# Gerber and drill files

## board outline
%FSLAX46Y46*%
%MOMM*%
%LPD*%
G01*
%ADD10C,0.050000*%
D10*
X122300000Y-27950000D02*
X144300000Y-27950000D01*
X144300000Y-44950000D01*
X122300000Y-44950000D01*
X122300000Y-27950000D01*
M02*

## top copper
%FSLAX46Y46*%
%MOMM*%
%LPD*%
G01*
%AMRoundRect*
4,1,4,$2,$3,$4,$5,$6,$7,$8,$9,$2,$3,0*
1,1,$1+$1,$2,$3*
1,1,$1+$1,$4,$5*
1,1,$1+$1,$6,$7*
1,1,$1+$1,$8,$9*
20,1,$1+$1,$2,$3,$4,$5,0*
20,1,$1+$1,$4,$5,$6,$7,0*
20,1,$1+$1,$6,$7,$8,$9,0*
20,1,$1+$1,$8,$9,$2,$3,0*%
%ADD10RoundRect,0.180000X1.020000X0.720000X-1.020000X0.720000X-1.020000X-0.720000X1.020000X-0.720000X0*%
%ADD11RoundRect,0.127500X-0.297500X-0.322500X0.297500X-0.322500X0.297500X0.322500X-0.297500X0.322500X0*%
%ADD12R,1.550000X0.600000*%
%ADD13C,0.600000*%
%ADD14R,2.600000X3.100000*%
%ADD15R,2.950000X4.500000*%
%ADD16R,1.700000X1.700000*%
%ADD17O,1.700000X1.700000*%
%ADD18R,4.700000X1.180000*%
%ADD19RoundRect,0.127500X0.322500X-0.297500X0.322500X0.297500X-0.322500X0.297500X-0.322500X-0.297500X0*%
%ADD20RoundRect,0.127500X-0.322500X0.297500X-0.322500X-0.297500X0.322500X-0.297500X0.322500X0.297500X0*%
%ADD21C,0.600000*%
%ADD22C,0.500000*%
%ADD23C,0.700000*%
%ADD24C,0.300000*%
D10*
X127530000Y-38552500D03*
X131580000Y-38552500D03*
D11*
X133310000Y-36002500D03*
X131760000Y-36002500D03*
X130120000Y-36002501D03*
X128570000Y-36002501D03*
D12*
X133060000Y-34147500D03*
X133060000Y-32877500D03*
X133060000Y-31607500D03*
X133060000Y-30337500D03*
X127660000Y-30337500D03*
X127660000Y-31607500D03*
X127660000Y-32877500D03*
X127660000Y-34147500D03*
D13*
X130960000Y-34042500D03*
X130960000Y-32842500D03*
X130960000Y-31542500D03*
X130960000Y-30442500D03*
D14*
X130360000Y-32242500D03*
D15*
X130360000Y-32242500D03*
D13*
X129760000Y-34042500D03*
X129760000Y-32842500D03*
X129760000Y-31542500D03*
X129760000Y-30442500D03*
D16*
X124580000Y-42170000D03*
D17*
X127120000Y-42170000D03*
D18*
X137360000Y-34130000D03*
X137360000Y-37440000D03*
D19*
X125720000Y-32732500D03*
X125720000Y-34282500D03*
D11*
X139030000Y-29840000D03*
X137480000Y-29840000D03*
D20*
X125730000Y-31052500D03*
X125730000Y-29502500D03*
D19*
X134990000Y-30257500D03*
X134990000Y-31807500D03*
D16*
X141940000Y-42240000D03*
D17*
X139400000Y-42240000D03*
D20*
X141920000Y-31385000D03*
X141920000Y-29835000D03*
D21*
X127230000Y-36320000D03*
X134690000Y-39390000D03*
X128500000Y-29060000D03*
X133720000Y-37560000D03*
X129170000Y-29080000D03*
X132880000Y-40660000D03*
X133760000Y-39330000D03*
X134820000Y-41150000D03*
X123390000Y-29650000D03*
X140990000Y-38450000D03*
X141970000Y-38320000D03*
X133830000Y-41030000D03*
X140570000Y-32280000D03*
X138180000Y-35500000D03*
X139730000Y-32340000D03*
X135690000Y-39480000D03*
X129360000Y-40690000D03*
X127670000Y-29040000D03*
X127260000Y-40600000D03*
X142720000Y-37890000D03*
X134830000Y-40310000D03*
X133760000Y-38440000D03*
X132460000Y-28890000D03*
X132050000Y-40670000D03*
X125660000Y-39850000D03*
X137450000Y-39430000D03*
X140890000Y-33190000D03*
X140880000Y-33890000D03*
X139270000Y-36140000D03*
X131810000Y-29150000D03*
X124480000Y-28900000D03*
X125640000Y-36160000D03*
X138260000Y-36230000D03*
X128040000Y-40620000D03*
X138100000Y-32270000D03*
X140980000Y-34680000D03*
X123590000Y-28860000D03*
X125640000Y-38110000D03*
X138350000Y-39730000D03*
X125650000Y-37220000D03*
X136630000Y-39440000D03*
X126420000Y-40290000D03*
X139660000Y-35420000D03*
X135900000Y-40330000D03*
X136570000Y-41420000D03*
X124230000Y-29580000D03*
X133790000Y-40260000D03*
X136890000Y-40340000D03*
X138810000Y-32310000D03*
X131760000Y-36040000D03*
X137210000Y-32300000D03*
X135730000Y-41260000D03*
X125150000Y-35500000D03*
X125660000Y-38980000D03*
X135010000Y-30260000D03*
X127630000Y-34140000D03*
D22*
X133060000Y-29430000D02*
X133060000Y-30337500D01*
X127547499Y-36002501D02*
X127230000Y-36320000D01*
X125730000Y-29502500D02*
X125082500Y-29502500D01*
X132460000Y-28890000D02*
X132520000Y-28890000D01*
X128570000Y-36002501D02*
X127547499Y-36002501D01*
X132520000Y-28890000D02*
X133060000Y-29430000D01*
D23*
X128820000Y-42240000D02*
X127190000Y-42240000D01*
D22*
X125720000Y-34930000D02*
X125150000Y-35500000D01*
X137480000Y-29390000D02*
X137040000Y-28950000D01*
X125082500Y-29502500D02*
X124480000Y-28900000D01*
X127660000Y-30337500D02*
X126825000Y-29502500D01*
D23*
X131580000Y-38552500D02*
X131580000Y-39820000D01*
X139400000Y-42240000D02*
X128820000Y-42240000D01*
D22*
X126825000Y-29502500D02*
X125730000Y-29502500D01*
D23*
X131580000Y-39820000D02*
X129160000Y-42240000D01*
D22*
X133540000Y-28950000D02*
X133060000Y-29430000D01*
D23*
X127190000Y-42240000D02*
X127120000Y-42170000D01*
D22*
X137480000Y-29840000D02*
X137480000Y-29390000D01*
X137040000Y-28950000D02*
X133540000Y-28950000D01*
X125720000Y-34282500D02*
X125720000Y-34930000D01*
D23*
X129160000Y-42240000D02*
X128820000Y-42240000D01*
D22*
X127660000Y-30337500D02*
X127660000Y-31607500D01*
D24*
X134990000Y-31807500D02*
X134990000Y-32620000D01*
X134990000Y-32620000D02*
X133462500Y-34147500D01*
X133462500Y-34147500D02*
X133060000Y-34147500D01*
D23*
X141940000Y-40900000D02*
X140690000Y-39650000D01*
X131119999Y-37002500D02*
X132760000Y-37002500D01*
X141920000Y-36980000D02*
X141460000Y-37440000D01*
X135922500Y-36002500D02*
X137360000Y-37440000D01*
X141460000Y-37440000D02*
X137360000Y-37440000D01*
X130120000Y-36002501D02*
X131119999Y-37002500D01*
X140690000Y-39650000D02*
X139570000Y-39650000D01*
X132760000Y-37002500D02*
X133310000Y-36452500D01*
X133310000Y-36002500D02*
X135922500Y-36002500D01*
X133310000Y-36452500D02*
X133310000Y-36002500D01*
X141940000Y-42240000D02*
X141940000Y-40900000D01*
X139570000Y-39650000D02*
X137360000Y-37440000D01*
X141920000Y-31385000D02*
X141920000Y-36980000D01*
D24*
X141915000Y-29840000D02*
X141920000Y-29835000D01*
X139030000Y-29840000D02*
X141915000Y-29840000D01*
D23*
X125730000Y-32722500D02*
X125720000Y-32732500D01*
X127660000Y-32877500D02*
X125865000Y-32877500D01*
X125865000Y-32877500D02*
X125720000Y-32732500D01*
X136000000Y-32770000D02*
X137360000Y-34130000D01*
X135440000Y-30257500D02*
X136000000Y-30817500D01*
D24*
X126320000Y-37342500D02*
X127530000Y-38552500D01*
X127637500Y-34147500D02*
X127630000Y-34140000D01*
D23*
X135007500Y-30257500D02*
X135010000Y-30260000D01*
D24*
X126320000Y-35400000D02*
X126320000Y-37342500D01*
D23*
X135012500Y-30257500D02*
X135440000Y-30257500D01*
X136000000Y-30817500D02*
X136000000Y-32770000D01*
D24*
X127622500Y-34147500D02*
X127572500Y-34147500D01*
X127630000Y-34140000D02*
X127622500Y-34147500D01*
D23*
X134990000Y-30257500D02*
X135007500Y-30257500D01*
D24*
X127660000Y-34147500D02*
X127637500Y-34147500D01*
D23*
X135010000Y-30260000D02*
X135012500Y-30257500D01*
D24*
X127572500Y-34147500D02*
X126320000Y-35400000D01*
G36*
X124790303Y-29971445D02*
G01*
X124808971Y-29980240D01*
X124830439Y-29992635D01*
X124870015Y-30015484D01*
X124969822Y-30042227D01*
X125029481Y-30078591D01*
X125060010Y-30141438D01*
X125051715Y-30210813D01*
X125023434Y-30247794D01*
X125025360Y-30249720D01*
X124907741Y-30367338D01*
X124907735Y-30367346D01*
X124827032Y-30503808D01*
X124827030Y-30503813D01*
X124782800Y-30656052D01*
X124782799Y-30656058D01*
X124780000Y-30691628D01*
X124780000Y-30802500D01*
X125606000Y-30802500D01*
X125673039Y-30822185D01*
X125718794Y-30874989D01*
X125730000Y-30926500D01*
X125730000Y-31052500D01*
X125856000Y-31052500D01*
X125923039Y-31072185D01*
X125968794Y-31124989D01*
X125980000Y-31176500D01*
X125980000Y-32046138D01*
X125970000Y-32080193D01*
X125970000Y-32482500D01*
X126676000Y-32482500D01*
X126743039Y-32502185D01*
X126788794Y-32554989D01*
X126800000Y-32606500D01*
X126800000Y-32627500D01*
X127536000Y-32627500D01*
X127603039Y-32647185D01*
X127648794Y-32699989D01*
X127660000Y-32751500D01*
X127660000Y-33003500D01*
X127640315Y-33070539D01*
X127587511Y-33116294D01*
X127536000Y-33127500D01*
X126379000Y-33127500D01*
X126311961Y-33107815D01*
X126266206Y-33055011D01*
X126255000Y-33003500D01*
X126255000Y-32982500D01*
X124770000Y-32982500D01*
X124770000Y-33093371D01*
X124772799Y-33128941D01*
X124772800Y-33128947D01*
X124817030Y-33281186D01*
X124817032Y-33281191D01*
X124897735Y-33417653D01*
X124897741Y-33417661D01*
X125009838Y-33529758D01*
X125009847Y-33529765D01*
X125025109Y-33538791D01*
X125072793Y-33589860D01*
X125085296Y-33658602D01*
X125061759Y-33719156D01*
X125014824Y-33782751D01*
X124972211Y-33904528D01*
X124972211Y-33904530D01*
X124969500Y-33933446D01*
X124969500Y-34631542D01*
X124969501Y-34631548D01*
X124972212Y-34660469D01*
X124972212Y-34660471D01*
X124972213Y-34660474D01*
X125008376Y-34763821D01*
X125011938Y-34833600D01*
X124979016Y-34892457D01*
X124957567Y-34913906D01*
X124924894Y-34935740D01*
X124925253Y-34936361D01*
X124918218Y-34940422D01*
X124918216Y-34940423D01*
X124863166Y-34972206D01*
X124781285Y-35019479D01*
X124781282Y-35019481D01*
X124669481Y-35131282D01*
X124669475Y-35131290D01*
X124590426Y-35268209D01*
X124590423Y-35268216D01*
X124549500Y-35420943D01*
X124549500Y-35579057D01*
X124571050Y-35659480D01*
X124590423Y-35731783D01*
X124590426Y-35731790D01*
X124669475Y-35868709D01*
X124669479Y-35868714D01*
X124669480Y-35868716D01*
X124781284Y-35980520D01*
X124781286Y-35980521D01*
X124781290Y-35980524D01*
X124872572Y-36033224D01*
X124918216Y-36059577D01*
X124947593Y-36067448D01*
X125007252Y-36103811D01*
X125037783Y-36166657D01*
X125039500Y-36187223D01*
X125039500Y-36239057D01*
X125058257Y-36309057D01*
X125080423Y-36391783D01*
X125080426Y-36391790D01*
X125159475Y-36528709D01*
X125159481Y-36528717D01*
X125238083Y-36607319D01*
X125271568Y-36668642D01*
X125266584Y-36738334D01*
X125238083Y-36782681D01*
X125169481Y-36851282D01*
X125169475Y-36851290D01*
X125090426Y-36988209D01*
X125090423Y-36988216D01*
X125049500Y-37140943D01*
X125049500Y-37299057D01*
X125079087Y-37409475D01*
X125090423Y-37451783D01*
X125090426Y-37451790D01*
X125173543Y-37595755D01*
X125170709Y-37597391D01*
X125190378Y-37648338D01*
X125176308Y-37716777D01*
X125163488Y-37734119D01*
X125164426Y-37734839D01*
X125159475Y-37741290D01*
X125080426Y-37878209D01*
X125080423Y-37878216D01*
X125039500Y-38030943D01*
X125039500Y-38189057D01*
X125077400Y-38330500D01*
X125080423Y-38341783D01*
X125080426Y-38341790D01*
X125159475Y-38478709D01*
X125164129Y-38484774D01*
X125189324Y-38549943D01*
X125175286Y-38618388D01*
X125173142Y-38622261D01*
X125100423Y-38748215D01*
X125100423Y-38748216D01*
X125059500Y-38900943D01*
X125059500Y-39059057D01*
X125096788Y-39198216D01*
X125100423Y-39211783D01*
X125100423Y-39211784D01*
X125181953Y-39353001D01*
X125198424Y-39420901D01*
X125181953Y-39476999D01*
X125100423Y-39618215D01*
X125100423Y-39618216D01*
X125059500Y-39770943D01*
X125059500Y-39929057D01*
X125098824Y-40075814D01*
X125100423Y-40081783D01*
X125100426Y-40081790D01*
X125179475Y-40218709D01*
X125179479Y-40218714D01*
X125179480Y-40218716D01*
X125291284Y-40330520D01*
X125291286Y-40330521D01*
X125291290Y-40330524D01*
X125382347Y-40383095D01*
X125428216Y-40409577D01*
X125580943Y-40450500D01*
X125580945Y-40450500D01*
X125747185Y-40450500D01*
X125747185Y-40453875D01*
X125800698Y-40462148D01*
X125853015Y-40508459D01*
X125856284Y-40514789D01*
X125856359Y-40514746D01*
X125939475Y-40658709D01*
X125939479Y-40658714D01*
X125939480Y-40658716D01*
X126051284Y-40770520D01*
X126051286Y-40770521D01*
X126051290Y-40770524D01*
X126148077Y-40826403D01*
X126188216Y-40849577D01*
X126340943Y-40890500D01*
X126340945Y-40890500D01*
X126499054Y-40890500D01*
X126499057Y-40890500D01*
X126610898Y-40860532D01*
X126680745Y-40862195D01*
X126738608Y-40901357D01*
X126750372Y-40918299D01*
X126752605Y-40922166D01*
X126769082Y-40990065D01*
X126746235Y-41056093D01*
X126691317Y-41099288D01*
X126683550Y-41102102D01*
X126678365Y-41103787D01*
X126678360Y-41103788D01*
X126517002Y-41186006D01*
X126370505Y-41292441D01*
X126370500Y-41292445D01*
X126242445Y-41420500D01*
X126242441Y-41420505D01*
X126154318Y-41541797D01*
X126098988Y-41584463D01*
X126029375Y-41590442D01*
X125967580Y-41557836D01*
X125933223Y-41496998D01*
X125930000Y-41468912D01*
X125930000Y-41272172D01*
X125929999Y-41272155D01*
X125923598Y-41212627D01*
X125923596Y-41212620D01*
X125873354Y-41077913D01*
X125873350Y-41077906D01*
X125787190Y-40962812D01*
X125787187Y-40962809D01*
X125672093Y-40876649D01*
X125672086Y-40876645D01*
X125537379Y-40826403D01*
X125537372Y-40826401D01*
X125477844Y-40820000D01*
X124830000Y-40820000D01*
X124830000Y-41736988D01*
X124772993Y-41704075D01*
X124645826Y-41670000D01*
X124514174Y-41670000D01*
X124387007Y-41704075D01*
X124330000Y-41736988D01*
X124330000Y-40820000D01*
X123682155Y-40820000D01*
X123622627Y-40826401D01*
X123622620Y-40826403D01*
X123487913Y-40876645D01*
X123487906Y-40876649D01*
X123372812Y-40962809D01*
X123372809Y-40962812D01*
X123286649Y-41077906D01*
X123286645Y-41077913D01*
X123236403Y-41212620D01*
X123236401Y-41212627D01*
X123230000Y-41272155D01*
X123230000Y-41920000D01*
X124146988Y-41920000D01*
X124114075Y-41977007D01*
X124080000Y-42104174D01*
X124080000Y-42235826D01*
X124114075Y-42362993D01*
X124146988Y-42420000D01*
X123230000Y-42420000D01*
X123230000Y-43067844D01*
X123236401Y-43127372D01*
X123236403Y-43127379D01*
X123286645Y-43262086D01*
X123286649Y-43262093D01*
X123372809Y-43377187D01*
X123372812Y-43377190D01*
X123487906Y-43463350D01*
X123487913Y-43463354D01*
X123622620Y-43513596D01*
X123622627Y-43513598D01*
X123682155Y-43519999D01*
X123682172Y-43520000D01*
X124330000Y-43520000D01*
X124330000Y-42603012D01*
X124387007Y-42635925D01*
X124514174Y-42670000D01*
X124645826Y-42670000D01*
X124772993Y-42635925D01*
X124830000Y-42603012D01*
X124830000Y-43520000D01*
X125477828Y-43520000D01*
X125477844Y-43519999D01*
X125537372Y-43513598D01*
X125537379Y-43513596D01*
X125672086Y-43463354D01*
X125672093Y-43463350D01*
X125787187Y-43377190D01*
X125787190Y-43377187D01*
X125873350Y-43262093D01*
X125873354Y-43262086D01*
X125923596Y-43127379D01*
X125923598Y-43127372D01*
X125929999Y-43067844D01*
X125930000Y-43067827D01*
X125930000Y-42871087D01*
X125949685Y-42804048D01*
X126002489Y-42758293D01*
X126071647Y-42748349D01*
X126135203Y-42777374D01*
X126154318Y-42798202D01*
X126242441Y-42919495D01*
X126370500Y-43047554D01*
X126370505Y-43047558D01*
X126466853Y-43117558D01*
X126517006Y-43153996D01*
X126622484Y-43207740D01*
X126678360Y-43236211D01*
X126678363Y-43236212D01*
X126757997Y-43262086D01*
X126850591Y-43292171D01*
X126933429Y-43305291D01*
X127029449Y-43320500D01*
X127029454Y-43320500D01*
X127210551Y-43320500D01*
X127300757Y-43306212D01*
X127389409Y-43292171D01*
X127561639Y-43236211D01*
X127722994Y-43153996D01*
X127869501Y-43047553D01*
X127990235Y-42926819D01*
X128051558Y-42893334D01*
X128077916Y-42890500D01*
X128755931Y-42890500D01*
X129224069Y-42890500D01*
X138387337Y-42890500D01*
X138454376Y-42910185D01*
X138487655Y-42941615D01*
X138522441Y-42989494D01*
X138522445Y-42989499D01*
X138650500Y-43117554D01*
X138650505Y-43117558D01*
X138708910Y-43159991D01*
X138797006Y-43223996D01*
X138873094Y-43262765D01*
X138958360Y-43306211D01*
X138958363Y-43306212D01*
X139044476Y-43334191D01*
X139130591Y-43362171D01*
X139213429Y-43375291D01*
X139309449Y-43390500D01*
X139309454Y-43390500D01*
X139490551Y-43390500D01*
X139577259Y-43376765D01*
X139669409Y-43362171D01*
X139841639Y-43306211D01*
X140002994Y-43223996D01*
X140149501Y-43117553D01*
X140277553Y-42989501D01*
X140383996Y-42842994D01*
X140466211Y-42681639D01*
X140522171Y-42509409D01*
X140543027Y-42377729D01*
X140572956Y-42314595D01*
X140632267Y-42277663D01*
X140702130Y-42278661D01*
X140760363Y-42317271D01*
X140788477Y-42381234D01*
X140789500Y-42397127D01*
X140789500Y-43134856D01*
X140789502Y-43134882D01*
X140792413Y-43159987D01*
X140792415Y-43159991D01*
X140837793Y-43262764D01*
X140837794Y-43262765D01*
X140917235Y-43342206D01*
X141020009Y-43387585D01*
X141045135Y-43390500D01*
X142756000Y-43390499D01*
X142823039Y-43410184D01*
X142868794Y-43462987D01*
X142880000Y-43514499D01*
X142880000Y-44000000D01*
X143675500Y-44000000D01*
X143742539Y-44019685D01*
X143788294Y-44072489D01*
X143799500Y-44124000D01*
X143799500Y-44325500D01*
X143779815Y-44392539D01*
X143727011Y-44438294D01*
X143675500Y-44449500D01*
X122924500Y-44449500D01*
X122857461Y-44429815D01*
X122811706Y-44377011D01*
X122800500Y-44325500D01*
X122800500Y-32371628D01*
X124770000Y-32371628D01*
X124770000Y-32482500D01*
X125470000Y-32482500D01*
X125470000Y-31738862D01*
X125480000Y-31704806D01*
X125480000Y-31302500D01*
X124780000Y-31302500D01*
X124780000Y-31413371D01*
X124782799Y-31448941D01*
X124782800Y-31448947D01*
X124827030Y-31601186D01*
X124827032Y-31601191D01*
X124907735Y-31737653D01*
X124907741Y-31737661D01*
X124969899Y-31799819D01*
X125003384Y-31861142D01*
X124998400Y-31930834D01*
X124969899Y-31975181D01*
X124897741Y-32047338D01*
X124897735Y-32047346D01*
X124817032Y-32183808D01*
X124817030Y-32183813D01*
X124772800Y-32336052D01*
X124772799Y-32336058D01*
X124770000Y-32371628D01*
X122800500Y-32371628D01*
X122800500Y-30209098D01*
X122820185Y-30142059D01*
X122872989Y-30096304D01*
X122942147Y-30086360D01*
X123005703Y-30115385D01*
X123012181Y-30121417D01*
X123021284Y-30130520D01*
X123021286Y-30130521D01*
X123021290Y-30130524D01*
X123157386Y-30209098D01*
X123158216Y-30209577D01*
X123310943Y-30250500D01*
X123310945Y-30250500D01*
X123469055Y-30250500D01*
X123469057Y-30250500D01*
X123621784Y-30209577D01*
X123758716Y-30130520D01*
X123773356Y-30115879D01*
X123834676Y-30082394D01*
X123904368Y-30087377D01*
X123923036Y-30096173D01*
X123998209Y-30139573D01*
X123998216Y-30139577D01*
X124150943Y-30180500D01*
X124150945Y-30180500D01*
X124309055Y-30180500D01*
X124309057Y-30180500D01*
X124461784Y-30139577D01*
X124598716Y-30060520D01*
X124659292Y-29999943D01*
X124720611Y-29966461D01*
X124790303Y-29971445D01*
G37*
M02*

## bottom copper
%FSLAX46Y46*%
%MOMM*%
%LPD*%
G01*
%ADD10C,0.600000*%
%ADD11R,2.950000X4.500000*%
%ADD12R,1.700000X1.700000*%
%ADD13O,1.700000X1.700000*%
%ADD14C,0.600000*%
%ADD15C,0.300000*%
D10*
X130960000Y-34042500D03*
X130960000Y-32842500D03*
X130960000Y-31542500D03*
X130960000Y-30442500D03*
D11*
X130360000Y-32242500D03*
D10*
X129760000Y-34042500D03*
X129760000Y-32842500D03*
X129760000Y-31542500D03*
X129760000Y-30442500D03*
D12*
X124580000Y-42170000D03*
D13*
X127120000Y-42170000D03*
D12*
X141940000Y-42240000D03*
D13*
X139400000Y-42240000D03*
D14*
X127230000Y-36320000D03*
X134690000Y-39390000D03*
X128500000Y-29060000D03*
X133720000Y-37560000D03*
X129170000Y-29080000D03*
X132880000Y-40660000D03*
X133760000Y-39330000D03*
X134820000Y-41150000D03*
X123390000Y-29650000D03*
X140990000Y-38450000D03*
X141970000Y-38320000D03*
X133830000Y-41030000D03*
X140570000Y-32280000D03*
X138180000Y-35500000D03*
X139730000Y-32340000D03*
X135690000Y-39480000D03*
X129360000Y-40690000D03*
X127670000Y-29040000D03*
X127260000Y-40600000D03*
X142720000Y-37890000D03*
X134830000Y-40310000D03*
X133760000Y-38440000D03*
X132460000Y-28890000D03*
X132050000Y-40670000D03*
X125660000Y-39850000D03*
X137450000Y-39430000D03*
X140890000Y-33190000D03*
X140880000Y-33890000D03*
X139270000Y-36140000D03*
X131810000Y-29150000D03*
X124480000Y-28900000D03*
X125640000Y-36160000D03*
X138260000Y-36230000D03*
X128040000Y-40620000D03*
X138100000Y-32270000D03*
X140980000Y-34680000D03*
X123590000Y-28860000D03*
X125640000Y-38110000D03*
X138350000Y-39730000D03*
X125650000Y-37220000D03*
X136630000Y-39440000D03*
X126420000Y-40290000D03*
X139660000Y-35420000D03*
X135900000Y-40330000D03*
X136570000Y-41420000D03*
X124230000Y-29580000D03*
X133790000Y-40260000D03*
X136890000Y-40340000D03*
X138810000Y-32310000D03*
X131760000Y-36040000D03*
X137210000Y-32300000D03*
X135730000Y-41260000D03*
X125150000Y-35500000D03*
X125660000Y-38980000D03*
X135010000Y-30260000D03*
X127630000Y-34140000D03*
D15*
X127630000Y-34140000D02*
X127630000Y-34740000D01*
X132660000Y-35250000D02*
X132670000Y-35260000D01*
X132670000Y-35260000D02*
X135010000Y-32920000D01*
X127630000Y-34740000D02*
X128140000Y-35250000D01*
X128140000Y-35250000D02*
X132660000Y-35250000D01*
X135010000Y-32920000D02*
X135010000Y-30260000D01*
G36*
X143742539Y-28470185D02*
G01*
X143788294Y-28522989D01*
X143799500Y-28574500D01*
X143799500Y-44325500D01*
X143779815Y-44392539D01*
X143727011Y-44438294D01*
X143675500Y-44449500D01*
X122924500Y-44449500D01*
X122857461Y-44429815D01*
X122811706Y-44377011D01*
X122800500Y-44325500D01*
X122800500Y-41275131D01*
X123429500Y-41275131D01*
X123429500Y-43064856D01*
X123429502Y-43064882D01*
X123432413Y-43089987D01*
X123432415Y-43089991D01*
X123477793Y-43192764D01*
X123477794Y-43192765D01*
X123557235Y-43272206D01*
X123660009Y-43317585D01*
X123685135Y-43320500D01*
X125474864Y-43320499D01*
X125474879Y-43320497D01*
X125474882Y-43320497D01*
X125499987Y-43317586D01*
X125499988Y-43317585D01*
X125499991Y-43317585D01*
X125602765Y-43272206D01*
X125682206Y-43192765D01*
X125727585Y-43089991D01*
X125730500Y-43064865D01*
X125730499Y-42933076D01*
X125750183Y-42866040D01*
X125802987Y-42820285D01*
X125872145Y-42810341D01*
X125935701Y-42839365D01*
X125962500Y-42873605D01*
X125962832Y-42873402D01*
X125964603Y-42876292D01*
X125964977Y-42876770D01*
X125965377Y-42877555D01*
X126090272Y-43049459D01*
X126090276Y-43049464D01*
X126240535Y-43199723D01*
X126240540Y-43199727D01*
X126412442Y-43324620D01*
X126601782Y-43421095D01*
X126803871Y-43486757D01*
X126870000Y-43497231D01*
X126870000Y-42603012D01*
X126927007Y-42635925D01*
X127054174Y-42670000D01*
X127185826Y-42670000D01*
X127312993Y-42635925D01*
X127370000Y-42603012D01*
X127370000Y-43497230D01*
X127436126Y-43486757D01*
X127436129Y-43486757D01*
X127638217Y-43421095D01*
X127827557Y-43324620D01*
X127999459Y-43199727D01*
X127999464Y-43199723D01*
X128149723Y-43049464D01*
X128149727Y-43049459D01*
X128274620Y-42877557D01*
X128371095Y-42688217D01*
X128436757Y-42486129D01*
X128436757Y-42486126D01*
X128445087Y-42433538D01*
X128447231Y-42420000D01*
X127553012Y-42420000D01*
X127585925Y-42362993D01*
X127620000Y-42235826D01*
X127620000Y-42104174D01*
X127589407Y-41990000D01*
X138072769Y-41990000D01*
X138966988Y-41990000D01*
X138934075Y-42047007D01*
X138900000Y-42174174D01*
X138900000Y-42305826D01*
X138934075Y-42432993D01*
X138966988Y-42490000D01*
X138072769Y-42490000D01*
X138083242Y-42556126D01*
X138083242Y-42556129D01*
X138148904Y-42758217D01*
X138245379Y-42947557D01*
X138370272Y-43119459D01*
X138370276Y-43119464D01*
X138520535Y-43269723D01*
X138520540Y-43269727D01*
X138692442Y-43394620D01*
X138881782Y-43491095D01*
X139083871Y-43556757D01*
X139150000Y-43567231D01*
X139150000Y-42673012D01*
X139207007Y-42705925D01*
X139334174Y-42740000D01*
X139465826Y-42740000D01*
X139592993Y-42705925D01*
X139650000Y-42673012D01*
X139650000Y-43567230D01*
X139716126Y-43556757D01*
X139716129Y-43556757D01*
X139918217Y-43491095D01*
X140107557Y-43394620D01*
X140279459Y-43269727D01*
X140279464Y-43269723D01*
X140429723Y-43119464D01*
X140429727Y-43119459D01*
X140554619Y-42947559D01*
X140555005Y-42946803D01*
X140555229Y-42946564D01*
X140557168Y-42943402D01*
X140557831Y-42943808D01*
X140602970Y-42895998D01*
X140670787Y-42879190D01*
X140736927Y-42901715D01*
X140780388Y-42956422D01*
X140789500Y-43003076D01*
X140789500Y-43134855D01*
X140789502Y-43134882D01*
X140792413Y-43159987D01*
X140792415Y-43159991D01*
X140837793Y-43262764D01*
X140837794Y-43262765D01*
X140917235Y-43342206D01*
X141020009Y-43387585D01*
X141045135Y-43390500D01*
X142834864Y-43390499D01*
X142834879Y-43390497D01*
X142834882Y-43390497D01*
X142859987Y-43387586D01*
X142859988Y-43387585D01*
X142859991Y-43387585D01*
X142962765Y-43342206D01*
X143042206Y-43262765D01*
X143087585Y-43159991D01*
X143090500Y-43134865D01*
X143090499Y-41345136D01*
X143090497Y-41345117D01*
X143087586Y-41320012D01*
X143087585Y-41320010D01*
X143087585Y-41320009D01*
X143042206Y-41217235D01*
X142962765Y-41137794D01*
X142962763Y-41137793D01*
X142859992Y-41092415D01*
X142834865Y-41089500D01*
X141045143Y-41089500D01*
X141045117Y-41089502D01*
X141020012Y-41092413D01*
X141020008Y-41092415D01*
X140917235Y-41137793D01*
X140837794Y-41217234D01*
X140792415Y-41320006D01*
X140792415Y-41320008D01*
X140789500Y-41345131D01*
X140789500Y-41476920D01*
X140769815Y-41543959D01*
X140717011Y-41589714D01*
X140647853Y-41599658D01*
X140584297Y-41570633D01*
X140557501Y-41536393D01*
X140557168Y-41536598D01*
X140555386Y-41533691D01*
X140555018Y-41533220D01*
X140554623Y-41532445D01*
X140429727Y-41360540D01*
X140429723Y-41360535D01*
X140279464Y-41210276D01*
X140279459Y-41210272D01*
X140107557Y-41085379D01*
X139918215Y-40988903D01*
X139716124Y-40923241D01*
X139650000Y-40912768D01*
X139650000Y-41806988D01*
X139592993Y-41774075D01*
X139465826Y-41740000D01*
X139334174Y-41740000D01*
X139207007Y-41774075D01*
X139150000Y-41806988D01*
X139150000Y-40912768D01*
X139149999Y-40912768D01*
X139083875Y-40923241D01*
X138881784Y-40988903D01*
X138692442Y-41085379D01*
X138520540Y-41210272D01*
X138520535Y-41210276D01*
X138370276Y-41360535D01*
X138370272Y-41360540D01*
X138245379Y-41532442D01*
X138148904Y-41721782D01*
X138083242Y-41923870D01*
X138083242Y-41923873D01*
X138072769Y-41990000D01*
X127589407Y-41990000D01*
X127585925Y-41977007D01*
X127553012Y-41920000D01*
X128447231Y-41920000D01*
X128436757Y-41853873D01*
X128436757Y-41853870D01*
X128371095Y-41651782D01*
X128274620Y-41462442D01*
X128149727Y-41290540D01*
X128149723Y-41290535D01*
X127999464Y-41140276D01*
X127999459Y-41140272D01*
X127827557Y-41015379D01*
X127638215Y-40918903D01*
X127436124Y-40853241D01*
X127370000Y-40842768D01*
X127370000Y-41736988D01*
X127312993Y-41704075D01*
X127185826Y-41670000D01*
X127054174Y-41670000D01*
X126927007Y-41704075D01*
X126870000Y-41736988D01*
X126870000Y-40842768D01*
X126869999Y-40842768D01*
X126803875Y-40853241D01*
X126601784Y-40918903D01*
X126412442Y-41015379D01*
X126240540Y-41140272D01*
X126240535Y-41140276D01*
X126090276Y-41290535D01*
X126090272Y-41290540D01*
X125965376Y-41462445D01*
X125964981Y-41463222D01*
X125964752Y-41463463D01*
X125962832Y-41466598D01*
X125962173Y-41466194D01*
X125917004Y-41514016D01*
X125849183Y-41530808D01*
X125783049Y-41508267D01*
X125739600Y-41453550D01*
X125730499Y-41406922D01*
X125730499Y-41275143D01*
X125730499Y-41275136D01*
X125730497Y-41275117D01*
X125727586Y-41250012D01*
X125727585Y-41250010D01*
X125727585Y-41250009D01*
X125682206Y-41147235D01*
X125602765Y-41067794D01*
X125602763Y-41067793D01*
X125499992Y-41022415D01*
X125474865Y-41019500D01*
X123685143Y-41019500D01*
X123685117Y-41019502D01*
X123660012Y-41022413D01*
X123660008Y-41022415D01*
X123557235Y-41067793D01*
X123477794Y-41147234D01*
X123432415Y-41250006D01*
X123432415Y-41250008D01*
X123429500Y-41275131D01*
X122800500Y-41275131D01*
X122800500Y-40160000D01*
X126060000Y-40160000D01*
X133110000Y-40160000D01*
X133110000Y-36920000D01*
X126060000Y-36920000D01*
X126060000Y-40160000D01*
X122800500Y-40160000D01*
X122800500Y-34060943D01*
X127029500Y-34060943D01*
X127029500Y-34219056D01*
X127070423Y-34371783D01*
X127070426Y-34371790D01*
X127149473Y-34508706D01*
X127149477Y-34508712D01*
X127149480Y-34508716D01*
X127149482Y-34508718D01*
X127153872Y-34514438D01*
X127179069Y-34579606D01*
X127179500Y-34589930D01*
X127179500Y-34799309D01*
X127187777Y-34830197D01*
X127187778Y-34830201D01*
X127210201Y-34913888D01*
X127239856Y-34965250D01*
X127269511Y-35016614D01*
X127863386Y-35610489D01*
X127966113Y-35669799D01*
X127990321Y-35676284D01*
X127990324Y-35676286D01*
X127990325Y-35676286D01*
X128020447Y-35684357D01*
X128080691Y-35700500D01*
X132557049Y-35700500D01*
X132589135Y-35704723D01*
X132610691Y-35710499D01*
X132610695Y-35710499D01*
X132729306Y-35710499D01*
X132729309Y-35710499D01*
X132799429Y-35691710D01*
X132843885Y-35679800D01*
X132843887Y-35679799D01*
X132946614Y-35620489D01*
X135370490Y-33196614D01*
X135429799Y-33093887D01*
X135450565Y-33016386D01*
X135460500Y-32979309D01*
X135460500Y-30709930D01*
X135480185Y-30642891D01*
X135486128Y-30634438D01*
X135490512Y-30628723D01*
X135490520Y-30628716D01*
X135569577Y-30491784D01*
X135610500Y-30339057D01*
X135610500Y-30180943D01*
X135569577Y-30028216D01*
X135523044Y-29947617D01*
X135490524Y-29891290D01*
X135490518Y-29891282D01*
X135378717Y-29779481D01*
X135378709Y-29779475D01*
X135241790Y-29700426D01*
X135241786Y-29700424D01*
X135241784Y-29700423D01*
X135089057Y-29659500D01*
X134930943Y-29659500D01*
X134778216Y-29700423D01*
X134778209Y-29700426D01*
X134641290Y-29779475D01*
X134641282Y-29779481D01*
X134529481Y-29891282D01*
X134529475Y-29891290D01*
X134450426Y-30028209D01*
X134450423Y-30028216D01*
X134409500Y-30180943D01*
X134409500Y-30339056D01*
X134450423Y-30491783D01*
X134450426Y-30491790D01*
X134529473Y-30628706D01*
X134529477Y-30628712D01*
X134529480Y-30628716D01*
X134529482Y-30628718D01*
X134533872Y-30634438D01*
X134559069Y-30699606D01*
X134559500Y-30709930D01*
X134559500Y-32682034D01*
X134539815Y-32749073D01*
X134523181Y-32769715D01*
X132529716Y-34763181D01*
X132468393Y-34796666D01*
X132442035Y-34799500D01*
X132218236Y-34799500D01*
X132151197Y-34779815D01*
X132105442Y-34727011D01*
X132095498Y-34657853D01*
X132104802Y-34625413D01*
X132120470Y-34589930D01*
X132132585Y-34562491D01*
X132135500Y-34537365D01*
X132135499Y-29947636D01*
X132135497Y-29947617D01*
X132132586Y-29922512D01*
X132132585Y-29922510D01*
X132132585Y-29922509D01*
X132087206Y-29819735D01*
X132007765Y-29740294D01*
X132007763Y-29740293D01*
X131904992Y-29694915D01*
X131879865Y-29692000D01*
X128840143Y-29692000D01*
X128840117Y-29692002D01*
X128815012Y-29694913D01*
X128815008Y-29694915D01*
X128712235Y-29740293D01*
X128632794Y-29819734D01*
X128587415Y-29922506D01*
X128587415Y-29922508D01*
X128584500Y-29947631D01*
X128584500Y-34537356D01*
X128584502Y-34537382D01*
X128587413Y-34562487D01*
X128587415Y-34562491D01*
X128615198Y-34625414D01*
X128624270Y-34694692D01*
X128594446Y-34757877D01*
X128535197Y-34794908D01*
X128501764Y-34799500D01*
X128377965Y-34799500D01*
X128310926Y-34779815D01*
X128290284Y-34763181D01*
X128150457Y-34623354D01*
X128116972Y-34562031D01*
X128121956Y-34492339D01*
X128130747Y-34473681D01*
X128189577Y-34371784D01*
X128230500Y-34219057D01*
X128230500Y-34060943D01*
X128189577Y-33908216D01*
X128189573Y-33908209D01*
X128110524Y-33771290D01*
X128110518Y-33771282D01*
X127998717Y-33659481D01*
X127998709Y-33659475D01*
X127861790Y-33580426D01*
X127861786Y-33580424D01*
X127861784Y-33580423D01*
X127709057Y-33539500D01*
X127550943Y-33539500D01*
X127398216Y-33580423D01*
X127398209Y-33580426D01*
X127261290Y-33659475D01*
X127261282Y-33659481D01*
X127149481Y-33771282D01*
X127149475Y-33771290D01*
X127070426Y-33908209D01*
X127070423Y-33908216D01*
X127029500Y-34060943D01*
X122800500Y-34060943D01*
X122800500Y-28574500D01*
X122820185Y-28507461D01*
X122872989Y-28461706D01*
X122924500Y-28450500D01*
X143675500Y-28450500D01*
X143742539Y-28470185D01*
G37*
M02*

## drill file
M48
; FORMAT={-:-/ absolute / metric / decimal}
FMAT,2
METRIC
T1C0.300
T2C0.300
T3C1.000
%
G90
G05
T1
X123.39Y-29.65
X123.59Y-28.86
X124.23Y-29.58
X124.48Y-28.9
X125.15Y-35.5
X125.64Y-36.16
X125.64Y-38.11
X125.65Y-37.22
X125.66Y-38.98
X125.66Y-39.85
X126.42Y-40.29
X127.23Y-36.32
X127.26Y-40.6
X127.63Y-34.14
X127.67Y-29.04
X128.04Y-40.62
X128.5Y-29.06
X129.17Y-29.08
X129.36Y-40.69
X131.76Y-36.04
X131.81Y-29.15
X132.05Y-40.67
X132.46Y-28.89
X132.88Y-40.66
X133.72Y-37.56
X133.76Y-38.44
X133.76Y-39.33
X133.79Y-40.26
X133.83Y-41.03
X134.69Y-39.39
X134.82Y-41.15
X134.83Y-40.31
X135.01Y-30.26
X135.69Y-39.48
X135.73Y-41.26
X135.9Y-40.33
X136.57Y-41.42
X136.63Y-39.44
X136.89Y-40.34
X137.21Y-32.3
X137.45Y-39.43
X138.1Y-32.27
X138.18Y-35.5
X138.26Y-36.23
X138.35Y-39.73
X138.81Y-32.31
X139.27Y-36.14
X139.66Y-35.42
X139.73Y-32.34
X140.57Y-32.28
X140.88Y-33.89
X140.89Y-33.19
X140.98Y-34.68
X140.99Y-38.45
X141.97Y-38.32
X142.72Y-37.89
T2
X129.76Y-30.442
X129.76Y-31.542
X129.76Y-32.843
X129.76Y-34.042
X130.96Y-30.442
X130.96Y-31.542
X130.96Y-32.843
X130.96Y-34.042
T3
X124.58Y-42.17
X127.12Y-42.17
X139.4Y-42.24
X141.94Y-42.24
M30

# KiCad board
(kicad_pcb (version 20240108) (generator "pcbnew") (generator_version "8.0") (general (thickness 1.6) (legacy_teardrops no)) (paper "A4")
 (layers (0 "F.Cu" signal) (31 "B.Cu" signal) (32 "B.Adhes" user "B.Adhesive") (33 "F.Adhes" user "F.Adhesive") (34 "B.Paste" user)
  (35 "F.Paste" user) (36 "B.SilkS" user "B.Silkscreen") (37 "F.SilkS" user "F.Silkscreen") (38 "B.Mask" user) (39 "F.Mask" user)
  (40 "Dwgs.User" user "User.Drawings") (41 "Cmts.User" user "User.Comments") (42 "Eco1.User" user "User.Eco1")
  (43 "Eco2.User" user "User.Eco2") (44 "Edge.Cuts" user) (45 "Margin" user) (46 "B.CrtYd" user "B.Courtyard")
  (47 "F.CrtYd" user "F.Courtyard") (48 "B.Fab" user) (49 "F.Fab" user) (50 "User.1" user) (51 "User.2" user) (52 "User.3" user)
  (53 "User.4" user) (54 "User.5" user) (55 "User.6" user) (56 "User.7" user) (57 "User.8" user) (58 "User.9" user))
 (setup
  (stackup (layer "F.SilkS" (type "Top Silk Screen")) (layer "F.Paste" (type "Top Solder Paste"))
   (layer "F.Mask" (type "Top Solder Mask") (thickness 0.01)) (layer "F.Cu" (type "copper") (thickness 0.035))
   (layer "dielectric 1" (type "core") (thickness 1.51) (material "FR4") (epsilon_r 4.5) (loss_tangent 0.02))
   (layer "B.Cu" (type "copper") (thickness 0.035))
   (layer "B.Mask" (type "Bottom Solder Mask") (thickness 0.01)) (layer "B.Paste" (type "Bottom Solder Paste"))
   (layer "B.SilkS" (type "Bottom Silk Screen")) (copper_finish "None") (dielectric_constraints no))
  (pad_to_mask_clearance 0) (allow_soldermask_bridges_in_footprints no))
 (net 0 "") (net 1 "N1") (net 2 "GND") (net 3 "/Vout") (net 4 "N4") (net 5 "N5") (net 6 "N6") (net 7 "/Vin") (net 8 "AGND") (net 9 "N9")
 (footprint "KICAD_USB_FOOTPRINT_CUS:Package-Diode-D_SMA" (layer "F.Cu") (at 129.63 38.5525 180)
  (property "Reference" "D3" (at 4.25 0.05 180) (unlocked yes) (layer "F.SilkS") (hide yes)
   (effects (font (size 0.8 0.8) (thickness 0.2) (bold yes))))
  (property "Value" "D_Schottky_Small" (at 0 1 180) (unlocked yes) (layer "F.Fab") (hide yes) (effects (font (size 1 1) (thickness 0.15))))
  (pad "1" smd roundrect (at 2.1 0 180) (size 2.4 1.8) (layers "F.Cu" "F.Paste" "F.Mask") (roundrect_rratio 0.1) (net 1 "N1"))
  (pad "2" smd roundrect (at -1.95 0 180) (size 2.4 1.8) (layers "F.Cu" "F.Paste" "F.Mask") (roundrect_rratio 0.1) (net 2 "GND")))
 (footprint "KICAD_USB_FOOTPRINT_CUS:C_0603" (layer "F.Cu") (at 132.535 36.0025 180)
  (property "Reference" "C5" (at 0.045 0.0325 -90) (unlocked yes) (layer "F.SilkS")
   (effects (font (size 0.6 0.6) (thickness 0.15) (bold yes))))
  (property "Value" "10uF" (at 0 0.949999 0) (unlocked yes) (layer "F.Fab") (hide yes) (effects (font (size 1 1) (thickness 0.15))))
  (pad "1" smd roundrect (at -0.775 0) (size 0.85 0.9) (layers "F.Cu" "F.Paste" "F.Mask") (roundrect_rratio 0.15) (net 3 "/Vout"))
  (pad "2" smd roundrect (at 0.775 0) (size 0.85 0.9) (layers "F.Cu" "F.Paste" "F.Mask") (roundrect_rratio 0.15) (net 2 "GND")))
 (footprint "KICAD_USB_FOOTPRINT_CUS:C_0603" (layer "F.Cu") (at 129.345 36.002501 180)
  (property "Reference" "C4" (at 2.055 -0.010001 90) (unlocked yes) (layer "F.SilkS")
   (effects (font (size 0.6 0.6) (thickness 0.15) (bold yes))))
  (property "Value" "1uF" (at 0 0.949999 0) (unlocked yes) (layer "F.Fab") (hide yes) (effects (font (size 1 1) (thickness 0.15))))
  (pad "1" smd roundrect (at -0.775 0) (size 0.85 0.9) (layers "F.Cu" "F.Paste" "F.Mask") (roundrect_rratio 0.15) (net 3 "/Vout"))
  (pad "2" smd roundrect (at 0.775 0) (size 0.85 0.9) (layers "F.Cu" "F.Paste" "F.Mask") (roundrect_rratio 0.15) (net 2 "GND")))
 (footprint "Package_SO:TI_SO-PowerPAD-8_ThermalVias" (layer "F.Cu") (at 130.36 32.2425 180)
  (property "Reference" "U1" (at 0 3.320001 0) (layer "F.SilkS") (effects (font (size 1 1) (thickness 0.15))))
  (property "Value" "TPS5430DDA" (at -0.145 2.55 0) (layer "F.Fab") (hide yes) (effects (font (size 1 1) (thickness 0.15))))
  (pad "1" smd rect (at -2.7 -1.905 180) (size 1.55 0.6) (layers "F.Cu" "F.Paste" "F.Mask") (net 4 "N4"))
  (pad "2" smd rect (at -2.7 -0.635 180) (size 1.55 0.6) (layers "F.Cu" "F.Paste" "F.Mask") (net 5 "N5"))
  (pad "3" smd rect (at -2.7 0.635 180) (size 1.55 0.6) (layers "F.Cu" "F.Paste" "F.Mask") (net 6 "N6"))
  (pad "4" smd rect (at -2.7 1.905 180) (size 1.55 0.6) (layers "F.Cu" "F.Paste" "F.Mask") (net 2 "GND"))
  (pad "5" smd rect (at 2.7 1.905 180) (size 1.55 0.6) (layers "F.Cu" "F.Paste" "F.Mask") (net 2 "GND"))
  (pad "6" smd rect (at 2.7 0.635 180) (size 1.55 0.6) (layers "F.Cu" "F.Paste" "F.Mask") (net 2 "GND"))
  (pad "7" smd rect (at 2.7 -0.635 180) (size 1.55 0.6) (layers "F.Cu" "F.Paste" "F.Mask") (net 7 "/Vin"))
  (pad "8" smd rect (at 2.7 -1.905 180) (size 1.55 0.6) (layers "F.Cu" "F.Paste" "F.Mask") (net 1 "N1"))
  (pad "9" thru_hole circle (at -0.6 -1.8 180) (size 0.6 0.6) (drill 0.3) (layers "*.Cu") (remove_unused_layers no) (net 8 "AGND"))
  (pad "9" thru_hole circle (at -0.6 -0.6 180) (size 0.6 0.6) (drill 0.3) (layers "*.Cu") (remove_unused_layers no) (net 8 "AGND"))
  (pad "9" thru_hole circle (at -0.6 0.7 180) (size 0.6 0.6) (drill 0.3) (layers "*.Cu") (remove_unused_layers no) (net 8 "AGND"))
  (pad "9" thru_hole circle (at -0.6 1.8 180) (size 0.6 0.6) (drill 0.3) (layers "*.Cu") (remove_unused_layers no) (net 8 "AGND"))
  (pad "9" smd rect (at 0 0 180) (size 2.6 3.1) (layers "F.Cu" "F.Paste" "F.Mask") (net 8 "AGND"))
  (pad "9" smd rect (at 0 0 180) (size 2.95 4.5) (layers "F.Cu") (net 8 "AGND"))
  (pad "9" smd rect (at 0 0 180) (size 2.95 4.5) (layers "B.Cu") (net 8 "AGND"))
  (pad "9" thru_hole circle (at 0.6 -1.8 180) (size 0.6 0.6) (drill 0.3) (layers "*.Cu") (remove_unused_layers no) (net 8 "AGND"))
  (pad "9" thru_hole circle (at 0.6 -0.6 180) (size 0.6 0.6) (drill 0.3) (layers "*.Cu") (remove_unused_layers no) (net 8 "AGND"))
  (pad "9" thru_hole circle (at 0.6 0.7 180) (size 0.6 0.6) (drill 0.3) (layers "*.Cu") (remove_unused_layers no) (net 8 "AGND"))
  (pad "9" thru_hole circle (at 0.6 1.8 180) (size 0.6 0.6) (drill 0.3) (layers "*.Cu") (remove_unused_layers no) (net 8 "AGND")))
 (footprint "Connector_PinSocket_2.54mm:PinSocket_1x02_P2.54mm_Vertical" (layer "F.Cu") (at 124.58 42.17 90)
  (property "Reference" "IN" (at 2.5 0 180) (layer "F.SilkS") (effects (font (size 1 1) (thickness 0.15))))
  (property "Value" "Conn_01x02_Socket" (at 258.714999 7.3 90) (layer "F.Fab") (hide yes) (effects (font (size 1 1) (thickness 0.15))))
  (pad "1" thru_hole rect (at 0 0 90) (size 1.7 1.7) (drill 1) (layers "*.Cu" "*.Mask") (remove_unused_layers no) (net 7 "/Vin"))
  (pad "2" thru_hole oval (at 0 2.54 90) (size 1.7 1.7) (drill 1) (layers "*.Cu" "*.Mask") (remove_unused_layers no) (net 2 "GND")))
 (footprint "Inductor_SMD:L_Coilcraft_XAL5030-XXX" (layer "F.Cu") (at 137.36 35.785 -90)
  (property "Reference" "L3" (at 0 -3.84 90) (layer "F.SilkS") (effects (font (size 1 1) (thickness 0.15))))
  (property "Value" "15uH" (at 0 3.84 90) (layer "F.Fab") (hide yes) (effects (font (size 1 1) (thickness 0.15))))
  (pad "1" smd rect (at -1.655 0 270) (size 1.18 4.7) (layers "F.Cu" "F.Paste" "F.Mask") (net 1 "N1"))
  (pad "2" smd rect (at 1.655 0 270) (size 1.18 4.7) (layers "F.Cu" "F.Paste" "F.Mask") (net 3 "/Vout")))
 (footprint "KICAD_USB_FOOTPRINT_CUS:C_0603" (layer "F.Cu") (at 125.72 33.5075 -90)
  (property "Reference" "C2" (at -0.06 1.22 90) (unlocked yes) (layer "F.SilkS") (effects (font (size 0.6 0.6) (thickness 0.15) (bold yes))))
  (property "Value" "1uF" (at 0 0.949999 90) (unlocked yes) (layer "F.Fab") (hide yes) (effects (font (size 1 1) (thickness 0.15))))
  (pad "1" smd roundrect (at -0.775 0 90) (size 0.85 0.9) (layers "F.Cu" "F.Paste" "F.Mask") (roundrect_rratio 0.15) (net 7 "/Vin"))
  (pad "2" smd roundrect (at 0.775 0 90) (size 0.85 0.9) (layers "F.Cu" "F.Paste" "F.Mask") (roundrect_rratio 0.15) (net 2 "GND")))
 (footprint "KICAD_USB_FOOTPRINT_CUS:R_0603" (layer "F.Cu") (at 138.255 29.84 180)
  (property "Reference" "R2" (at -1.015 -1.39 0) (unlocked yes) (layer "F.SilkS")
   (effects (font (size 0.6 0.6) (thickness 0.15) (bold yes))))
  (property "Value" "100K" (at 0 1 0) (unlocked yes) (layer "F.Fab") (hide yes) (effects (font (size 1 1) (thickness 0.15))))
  (pad "1" smd roundrect (at -0.775 0) (size 0.85 0.9) (layers "F.Cu" "F.Paste" "F.Mask") (roundrect_rratio 0.15) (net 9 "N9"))
  (pad "2" smd roundrect (at 0.775 0) (size 0.85 0.9) (layers "F.Cu" "F.Paste" "F.Mask") (roundrect_rratio 0.15) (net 2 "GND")))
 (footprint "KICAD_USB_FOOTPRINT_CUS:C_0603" (layer "F.Cu") (at 125.73 30.2775 90)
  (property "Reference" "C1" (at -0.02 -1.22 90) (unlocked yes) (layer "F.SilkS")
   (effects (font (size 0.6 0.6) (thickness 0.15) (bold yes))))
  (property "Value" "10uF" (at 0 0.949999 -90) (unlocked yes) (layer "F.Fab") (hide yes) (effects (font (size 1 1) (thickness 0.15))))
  (pad "1" smd roundrect (at -0.775 0 270) (size 0.85 0.9) (layers "F.Cu" "F.Paste" "F.Mask") (roundrect_rratio 0.15) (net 7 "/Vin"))
  (pad "2" smd roundrect (at 0.775 0 270) (size 0.85 0.9) (layers "F.Cu" "F.Paste" "F.Mask") (roundrect_rratio 0.15) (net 2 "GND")))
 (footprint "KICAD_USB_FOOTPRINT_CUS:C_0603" (layer "F.Cu") (at 134.99 31.0325 -90)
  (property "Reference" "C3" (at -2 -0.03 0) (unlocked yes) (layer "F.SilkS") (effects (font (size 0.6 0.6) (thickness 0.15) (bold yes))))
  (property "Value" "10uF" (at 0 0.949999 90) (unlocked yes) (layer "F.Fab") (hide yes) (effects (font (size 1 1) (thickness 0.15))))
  (pad "1" smd roundrect (at -0.775 0 90) (size 0.85 0.9) (layers "F.Cu" "F.Paste" "F.Mask") (roundrect_rratio 0.15) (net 1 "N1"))
  (pad "2" smd roundrect (at 0.775 0 90) (size 0.85 0.9) (layers "F.Cu" "F.Paste" "F.Mask") (roundrect_rratio 0.15) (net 4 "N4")))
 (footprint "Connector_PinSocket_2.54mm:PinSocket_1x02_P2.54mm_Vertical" (layer "F.Cu") (at 141.94 42.24 -90)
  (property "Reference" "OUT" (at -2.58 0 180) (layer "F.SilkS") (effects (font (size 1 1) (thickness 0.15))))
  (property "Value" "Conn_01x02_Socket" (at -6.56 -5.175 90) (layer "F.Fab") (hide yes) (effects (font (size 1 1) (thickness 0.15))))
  (pad "1" thru_hole rect (at 0 0 270) (size 1.7 1.7) (drill 1) (layers "*.Cu" "*.Mask") (remove_unused_layers no) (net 3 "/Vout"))
  (pad "2" thru_hole oval (at 0 2.54 270) (size 1.7 1.7) (drill 1) (layers "*.Cu" "*.Mask") (remove_unused_layers no) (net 2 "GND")))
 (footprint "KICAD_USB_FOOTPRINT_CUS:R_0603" (layer "F.Cu") (at 141.92 30.61 90)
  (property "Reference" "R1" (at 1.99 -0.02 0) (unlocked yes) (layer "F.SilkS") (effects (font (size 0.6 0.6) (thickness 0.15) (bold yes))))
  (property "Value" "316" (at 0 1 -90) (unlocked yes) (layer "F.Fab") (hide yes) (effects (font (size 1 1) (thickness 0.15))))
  (pad "1" smd roundrect (at -0.775 0 270) (size 0.85 0.9) (layers "F.Cu" "F.Paste" "F.Mask") (roundrect_rratio 0.15) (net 3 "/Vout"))
  (pad "2" smd roundrect (at 0.775 0 270) (size 0.85 0.9) (layers "F.Cu" "F.Paste" "F.Mask") (roundrect_rratio 0.15) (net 9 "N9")))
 (gr_rect (start 122.3 27.95) (end 144.3 44.95) (stroke (width 0.05) (type default)) (fill none) (layer "Edge.Cuts"))
 (segment (start 133.06 29.43) (end 133.06 30.3375) (width 0.5) (layer "F.Cu") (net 2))
 (segment (start 127.547499 36.002501) (end 127.23 36.32) (width 0.5) (layer "F.Cu") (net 2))
 (segment (start 125.73 29.5025) (end 125.0825 29.5025) (width 0.5) (layer "F.Cu") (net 2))
 (segment (start 132.46 28.89) (end 132.52 28.89) (width 0.5) (layer "F.Cu") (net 2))
 (segment (start 128.57 36.002501) (end 127.547499 36.002501) (width 0.5) (layer "F.Cu") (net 2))
 (segment (start 132.52 28.89) (end 133.06 29.43) (width 0.5) (layer "F.Cu") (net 2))
 (segment (start 128.82 42.24) (end 127.19 42.24) (width 0.7) (layer "F.Cu") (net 2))
 (segment (start 125.72 34.93) (end 125.15 35.5) (width 0.5) (layer "F.Cu") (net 2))
 (segment (start 137.48 29.39) (end 137.04 28.95) (width 0.5) (layer "F.Cu") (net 2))
 (segment (start 125.0825 29.5025) (end 124.48 28.9) (width 0.5) (layer "F.Cu") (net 2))
 (segment (start 127.66 30.3375) (end 126.825 29.5025) (width 0.5) (layer "F.Cu") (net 2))
 (segment (start 131.58 38.5525) (end 131.58 39.82) (width 0.7) (layer "F.Cu") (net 2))
 (segment (start 139.4 42.24) (end 128.82 42.24) (width 0.7) (layer "F.Cu") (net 2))
 (segment (start 126.825 29.5025) (end 125.73 29.5025) (width 0.5) (layer "F.Cu") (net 2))
 (segment (start 131.58 39.82) (end 129.16 42.24) (width 0.7) (layer "F.Cu") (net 2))
 (segment (start 133.54 28.95) (end 133.06 29.43) (width 0.5) (layer "F.Cu") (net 2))
 (segment (start 127.19 42.24) (end 127.12 42.17) (width 0.7) (layer "F.Cu") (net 2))
 (segment (start 137.48 29.84) (end 137.48 29.39) (width 0.5) (layer "F.Cu") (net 2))
 (segment (start 137.04 28.95) (end 133.54 28.95) (width 0.5) (layer "F.Cu") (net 2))
 (segment (start 125.72 34.2825) (end 125.72 34.93) (width 0.5) (layer "F.Cu") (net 2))
 (segment (start 129.16 42.24) (end 128.82 42.24) (width 0.7) (layer "F.Cu") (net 2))
 (segment (start 127.66 30.3375) (end 127.66 31.6075) (width 0.5) (layer "F.Cu") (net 2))
 (via (at 127.23 36.32) (size 0.6) (drill 0.3) (layers "F.Cu" "B.Cu") (free yes) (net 2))
 (via (at 134.69 39.39) (size 0.6) (drill 0.3) (layers "F.Cu" "B.Cu") (free yes) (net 2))
 (via (at 128.5 29.06) (size 0.6) (drill 0.3) (layers "F.Cu" "B.Cu") (free yes) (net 2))
 (via (at 133.72 37.56) (size 0.6) (drill 0.3) (layers "F.Cu" "B.Cu") (free yes) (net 2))
 (via (at 129.17 29.08) (size 0.6) (drill 0.3) (layers "F.Cu" "B.Cu") (free yes) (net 2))
 (via (at 132.88 40.66) (size 0.6) (drill 0.3) (layers "F.Cu" "B.Cu") (free yes) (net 2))
 (via (at 133.76 39.33) (size 0.6) (drill 0.3) (layers "F.Cu" "B.Cu") (free yes) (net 2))
 (via (at 134.82 41.15) (size 0.6) (drill 0.3) (layers "F.Cu" "B.Cu") (free yes) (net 2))
 (via (at 123.39 29.65) (size 0.6) (drill 0.3) (layers "F.Cu" "B.Cu") (free yes) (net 2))
 (via (at 140.99 38.45) (size 0.6) (drill 0.3) (layers "F.Cu" "B.Cu") (free yes) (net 2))
 (via (at 141.97 38.32) (size 0.6) (drill 0.3) (layers "F.Cu" "B.Cu") (free yes) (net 2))
 (via (at 133.83 41.03) (size 0.6) (drill 0.3) (layers "F.Cu" "B.Cu") (free yes) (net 2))
 (via (at 140.57 32.28) (size 0.6) (drill 0.3) (layers "F.Cu" "B.Cu") (free yes) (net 2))
 (via (at 138.18 35.5) (size 0.6) (drill 0.3) (layers "F.Cu" "B.Cu") (free yes) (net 2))
 (via (at 139.73 32.34) (size 0.6) (drill 0.3) (layers "F.Cu" "B.Cu") (free yes) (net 2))
 (via (at 135.69 39.48) (size 0.6) (drill 0.3) (layers "F.Cu" "B.Cu") (free yes) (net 2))
 (via (at 129.36 40.69) (size 0.6) (drill 0.3) (layers "F.Cu" "B.Cu") (free yes) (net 2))
 (via (at 127.67 29.04) (size 0.6) (drill 0.3) (layers "F.Cu" "B.Cu") (free yes) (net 2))
 (via (at 127.26 40.6) (size 0.6) (drill 0.3) (layers "F.Cu" "B.Cu") (free yes) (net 2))
 (via (at 142.72 37.89) (size 0.6) (drill 0.3) (layers "F.Cu" "B.Cu") (free yes) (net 2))
 (via (at 134.83 40.31) (size 0.6) (drill 0.3) (layers "F.Cu" "B.Cu") (free yes) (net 2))
 (via (at 133.76 38.44) (size 0.6) (drill 0.3) (layers "F.Cu" "B.Cu") (free yes) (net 2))
 (via (at 132.46 28.89) (size 0.6) (drill 0.3) (layers "F.Cu" "B.Cu") (free yes) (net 2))
 (via (at 132.05 40.67) (size 0.6) (drill 0.3) (layers "F.Cu" "B.Cu") (free yes) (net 2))
 (via (at 125.66 39.85) (size 0.6) (drill 0.3) (layers "F.Cu" "B.Cu") (free yes) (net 2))
 (via (at 137.45 39.43) (size 0.6) (drill 0.3) (layers "F.Cu" "B.Cu") (free yes) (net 2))
 (via (at 140.89 33.19) (size 0.6) (drill 0.3) (layers "F.Cu" "B.Cu") (free yes) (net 2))
 (via (at 140.88 33.89) (size 0.6) (drill 0.3) (layers "F.Cu" "B.Cu") (free yes) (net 2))
 (via (at 139.27 36.14) (size 0.6) (drill 0.3) (layers "F.Cu" "B.Cu") (free yes) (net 2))
 (via (at 131.81 29.15) (size 0.6) (drill 0.3) (layers "F.Cu" "B.Cu") (free yes) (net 2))
 (via (at 124.48 28.9) (size 0.6) (drill 0.3) (layers "F.Cu" "B.Cu") (free yes) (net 2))
 (via (at 125.64 36.16) (size 0.6) (drill 0.3) (layers "F.Cu" "B.Cu") (free yes) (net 2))
 (via (at 138.26 36.23) (size 0.6) (drill 0.3) (layers "F.Cu" "B.Cu") (free yes) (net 2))
 (via (at 128.04 40.62) (size 0.6) (drill 0.3) (layers "F.Cu" "B.Cu") (free yes) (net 2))
 (via (at 138.1 32.27) (size 0.6) (drill 0.3) (layers "F.Cu" "B.Cu") (free yes) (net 2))
 (via (at 140.98 34.68) (size 0.6) (drill 0.3) (layers "F.Cu" "B.Cu") (free yes) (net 2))
 (via (at 123.59 28.86) (size 0.6) (drill 0.3) (layers "F.Cu" "B.Cu") (free yes) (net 2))
 (via (at 125.64 38.11) (size 0.6) (drill 0.3) (layers "F.Cu" "B.Cu") (free yes) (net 2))
 (via (at 138.35 39.73) (size 0.6) (drill 0.3) (layers "F.Cu" "B.Cu") (free yes) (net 2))
 (via (at 125.65 37.22) (size 0.6) (drill 0.3) (layers "F.Cu" "B.Cu") (free yes) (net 2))
 (via (at 136.63 39.44) (size 0.6) (drill 0.3) (layers "F.Cu" "B.Cu") (free yes) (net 2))
 (via (at 126.42 40.29) (size 0.6) (drill 0.3) (layers "F.Cu" "B.Cu") (free yes) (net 2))
 (via (at 139.66 35.42) (size 0.6) (drill 0.3) (layers "F.Cu" "B.Cu") (free yes) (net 2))
 (via (at 135.9 40.33) (size 0.6) (drill 0.3) (layers "F.Cu" "B.Cu") (free yes) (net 2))
 (via (at 136.57 41.42) (size 0.6) (drill 0.3) (layers "F.Cu" "B.Cu") (free yes) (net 2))
 (via (at 124.23 29.58) (size 0.6) (drill 0.3) (layers "F.Cu" "B.Cu") (free yes) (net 2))
 (via (at 133.79 40.26) (size 0.6) (drill 0.3) (layers "F.Cu" "B.Cu") (free yes) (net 2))
 (via (at 136.89 40.34) (size 0.6) (drill 0.3) (layers "F.Cu" "B.Cu") (free yes) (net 2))
 (via (at 138.81 32.31) (size 0.6) (drill 0.3) (layers "F.Cu" "B.Cu") (free yes) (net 2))
 (via (at 131.76 36.04) (size 0.6) (drill 0.3) (layers "F.Cu" "B.Cu") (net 2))
 (via (at 137.21 32.3) (size 0.6) (drill 0.3) (layers "F.Cu" "B.Cu") (free yes) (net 2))
 (via (at 135.73 41.26) (size 0.6) (drill 0.3) (layers "F.Cu" "B.Cu") (free yes) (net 2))
 (via (at 125.15 35.5) (size 0.6) (drill 0.3) (layers "F.Cu" "B.Cu") (free yes) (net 2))
 (via (at 125.66 38.98) (size 0.6) (drill 0.3) (layers "F.Cu" "B.Cu") (free yes) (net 2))
 (segment (start 134.99 31.8075) (end 134.99 32.62) (width 0.3) (layer "F.Cu") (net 4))
 (segment (start 134.99 32.62) (end 133.4625 34.1475) (width 0.3) (layer "F.Cu") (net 4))
 (segment (start 133.4625 34.1475) (end 133.06 34.1475) (width 0.3) (layer "F.Cu") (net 4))
 (segment (start 141.94 40.9) (end 140.69 39.65) (width 0.7) (layer "F.Cu") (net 3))
 (segment (start 131.119999 37.0025) (end 132.76 37.0025) (width 0.7) (layer "F.Cu") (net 3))
 (segment (start 141.92 36.98) (end 141.46 37.44) (width 0.7) (layer "F.Cu") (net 3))
 (segment (start 135.9225 36.0025) (end 137.36 37.44) (width 0.7) (layer "F.Cu") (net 3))
 (segment (start 141.46 37.44) (end 137.36 37.44) (width 0.7) (layer "F.Cu") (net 3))
 (segment (start 130.12 36.002501) (end 131.119999 37.0025) (width 0.7) (layer "F.Cu") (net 3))
 (segment (start 140.69 39.65) (end 139.57 39.65) (width 0.7) (layer "F.Cu") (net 3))
 (segment (start 132.76 37.0025) (end 133.31 36.4525) (width 0.7) (layer "F.Cu") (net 3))
 (segment (start 133.31 36.0025) (end 135.9225 36.0025) (width 0.7) (layer "F.Cu") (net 3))
 (segment (start 133.31 36.4525) (end 133.31 36.0025) (width 0.7) (layer "F.Cu") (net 3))
 (segment (start 141.94 42.24) (end 141.94 40.9) (width 0.7) (layer "F.Cu") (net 3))
 (segment (start 139.57 39.65) (end 137.36 37.44) (width 0.7) (layer "F.Cu") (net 3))
 (segment (start 141.92 31.385) (end 141.92 36.98) (width 0.7) (layer "F.Cu") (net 3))
 (segment (start 141.915 29.84) (end 141.92 29.835) (width 0.3) (layer "F.Cu") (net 9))
 (segment (start 139.03 29.84) (end 141.915 29.84) (width 0.3) (layer "F.Cu") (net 9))
 (segment (start 125.73 32.7225) (end 125.72 32.7325) (width 0.7) (layer "F.Cu") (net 7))
 (segment (start 127.66 32.8775) (end 125.865 32.8775) (width 0.7) (layer "F.Cu") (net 7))
 (segment (start 125.865 32.8775) (end 125.72 32.7325) (width 0.7) (layer "F.Cu") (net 7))
 (segment (start 136 32.77) (end 137.36 34.13) (width 0.7) (layer "F.Cu") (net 1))
 (segment (start 135.44 30.2575) (end 136 30.8175) (width 0.7) (layer "F.Cu") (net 1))
 (segment (start 126.32 37.3425) (end 127.53 38.5525) (width 0.3) (layer "F.Cu") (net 1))
 (segment (start 127.6375 34.1475) (end 127.63 34.14) (width 0.3) (layer "F.Cu") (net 1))
 (segment (start 135.0075 30.2575) (end 135.01 30.26) (width 0.7) (layer "F.Cu") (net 1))
 (segment (start 126.32 35.4) (end 126.32 37.3425) (width 0.3) (layer "F.Cu") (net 1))
 (segment (start 135.0125 30.2575) (end 135.44 30.2575) (width 0.7) (layer "F.Cu") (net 1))
 (segment (start 136 30.8175) (end 136 32.77) (width 0.7) (layer "F.Cu") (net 1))
 (segment (start 127.6225 34.1475) (end 127.5725 34.1475) (width 0.3) (layer "F.Cu") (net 1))
 (segment (start 127.63 34.14) (end 127.6225 34.1475) (width 0.3) (layer "F.Cu") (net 1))
 (segment (start 134.99 30.2575) (end 135.0075 30.2575) (width 0.7) (layer "F.Cu") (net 1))
 (segment (start 127.66 34.1475) (end 127.6375 34.1475) (width 0.3) (layer "F.Cu") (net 1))
 (segment (start 135.01 30.26) (end 135.0125 30.2575) (width 0.7) (layer "F.Cu") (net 1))
 (segment (start 127.5725 34.1475) (end 126.32 35.4) (width 0.3) (layer "F.Cu") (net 1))
 (via (at 135.01 30.26) (size 0.6) (drill 0.3) (layers "F.Cu" "B.Cu") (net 1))
 (via (at 127.63 34.14) (size 0.6) (drill 0.3) (layers "F.Cu" "B.Cu") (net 1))
 (segment (start 127.63 34.14) (end 127.63 34.74) (width 0.3) (layer "B.Cu") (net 1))
 (segment (start 132.66 35.25) (end 132.67 35.26) (width 0.3) (layer "B.Cu") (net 1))
 (segment (start 132.67 35.26) (end 135.01 32.92) (width 0.3) (layer "B.Cu") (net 1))
 (segment (start 127.63 34.74) (end 128.14 35.25) (width 0.3) (layer "B.Cu") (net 1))
 (segment (start 128.14 35.25) (end 132.66 35.25) (width 0.3) (layer "B.Cu") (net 1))
 (segment (start 135.01 32.92) (end 135.01 30.26) (width 0.3) (layer "B.Cu") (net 1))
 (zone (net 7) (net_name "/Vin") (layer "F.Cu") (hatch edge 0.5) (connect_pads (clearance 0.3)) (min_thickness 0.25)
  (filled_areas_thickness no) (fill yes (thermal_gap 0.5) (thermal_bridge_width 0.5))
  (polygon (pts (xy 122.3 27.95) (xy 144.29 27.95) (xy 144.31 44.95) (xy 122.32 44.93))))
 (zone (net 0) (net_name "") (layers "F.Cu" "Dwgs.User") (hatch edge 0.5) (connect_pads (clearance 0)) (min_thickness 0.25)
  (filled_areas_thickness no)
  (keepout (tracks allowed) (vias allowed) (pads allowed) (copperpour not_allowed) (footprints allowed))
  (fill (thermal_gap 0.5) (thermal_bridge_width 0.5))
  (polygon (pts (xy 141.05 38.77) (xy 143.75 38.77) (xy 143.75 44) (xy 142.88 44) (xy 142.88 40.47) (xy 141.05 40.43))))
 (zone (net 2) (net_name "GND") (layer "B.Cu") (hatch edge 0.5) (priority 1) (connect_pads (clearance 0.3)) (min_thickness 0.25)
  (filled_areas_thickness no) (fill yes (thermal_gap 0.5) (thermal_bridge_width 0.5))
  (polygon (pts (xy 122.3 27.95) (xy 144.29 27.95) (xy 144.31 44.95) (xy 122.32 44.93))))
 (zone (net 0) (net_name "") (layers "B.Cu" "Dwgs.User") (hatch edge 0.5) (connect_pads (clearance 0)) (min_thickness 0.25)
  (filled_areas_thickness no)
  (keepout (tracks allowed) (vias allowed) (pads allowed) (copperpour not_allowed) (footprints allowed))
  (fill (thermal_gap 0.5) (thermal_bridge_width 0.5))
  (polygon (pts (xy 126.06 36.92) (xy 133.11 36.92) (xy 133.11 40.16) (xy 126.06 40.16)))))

